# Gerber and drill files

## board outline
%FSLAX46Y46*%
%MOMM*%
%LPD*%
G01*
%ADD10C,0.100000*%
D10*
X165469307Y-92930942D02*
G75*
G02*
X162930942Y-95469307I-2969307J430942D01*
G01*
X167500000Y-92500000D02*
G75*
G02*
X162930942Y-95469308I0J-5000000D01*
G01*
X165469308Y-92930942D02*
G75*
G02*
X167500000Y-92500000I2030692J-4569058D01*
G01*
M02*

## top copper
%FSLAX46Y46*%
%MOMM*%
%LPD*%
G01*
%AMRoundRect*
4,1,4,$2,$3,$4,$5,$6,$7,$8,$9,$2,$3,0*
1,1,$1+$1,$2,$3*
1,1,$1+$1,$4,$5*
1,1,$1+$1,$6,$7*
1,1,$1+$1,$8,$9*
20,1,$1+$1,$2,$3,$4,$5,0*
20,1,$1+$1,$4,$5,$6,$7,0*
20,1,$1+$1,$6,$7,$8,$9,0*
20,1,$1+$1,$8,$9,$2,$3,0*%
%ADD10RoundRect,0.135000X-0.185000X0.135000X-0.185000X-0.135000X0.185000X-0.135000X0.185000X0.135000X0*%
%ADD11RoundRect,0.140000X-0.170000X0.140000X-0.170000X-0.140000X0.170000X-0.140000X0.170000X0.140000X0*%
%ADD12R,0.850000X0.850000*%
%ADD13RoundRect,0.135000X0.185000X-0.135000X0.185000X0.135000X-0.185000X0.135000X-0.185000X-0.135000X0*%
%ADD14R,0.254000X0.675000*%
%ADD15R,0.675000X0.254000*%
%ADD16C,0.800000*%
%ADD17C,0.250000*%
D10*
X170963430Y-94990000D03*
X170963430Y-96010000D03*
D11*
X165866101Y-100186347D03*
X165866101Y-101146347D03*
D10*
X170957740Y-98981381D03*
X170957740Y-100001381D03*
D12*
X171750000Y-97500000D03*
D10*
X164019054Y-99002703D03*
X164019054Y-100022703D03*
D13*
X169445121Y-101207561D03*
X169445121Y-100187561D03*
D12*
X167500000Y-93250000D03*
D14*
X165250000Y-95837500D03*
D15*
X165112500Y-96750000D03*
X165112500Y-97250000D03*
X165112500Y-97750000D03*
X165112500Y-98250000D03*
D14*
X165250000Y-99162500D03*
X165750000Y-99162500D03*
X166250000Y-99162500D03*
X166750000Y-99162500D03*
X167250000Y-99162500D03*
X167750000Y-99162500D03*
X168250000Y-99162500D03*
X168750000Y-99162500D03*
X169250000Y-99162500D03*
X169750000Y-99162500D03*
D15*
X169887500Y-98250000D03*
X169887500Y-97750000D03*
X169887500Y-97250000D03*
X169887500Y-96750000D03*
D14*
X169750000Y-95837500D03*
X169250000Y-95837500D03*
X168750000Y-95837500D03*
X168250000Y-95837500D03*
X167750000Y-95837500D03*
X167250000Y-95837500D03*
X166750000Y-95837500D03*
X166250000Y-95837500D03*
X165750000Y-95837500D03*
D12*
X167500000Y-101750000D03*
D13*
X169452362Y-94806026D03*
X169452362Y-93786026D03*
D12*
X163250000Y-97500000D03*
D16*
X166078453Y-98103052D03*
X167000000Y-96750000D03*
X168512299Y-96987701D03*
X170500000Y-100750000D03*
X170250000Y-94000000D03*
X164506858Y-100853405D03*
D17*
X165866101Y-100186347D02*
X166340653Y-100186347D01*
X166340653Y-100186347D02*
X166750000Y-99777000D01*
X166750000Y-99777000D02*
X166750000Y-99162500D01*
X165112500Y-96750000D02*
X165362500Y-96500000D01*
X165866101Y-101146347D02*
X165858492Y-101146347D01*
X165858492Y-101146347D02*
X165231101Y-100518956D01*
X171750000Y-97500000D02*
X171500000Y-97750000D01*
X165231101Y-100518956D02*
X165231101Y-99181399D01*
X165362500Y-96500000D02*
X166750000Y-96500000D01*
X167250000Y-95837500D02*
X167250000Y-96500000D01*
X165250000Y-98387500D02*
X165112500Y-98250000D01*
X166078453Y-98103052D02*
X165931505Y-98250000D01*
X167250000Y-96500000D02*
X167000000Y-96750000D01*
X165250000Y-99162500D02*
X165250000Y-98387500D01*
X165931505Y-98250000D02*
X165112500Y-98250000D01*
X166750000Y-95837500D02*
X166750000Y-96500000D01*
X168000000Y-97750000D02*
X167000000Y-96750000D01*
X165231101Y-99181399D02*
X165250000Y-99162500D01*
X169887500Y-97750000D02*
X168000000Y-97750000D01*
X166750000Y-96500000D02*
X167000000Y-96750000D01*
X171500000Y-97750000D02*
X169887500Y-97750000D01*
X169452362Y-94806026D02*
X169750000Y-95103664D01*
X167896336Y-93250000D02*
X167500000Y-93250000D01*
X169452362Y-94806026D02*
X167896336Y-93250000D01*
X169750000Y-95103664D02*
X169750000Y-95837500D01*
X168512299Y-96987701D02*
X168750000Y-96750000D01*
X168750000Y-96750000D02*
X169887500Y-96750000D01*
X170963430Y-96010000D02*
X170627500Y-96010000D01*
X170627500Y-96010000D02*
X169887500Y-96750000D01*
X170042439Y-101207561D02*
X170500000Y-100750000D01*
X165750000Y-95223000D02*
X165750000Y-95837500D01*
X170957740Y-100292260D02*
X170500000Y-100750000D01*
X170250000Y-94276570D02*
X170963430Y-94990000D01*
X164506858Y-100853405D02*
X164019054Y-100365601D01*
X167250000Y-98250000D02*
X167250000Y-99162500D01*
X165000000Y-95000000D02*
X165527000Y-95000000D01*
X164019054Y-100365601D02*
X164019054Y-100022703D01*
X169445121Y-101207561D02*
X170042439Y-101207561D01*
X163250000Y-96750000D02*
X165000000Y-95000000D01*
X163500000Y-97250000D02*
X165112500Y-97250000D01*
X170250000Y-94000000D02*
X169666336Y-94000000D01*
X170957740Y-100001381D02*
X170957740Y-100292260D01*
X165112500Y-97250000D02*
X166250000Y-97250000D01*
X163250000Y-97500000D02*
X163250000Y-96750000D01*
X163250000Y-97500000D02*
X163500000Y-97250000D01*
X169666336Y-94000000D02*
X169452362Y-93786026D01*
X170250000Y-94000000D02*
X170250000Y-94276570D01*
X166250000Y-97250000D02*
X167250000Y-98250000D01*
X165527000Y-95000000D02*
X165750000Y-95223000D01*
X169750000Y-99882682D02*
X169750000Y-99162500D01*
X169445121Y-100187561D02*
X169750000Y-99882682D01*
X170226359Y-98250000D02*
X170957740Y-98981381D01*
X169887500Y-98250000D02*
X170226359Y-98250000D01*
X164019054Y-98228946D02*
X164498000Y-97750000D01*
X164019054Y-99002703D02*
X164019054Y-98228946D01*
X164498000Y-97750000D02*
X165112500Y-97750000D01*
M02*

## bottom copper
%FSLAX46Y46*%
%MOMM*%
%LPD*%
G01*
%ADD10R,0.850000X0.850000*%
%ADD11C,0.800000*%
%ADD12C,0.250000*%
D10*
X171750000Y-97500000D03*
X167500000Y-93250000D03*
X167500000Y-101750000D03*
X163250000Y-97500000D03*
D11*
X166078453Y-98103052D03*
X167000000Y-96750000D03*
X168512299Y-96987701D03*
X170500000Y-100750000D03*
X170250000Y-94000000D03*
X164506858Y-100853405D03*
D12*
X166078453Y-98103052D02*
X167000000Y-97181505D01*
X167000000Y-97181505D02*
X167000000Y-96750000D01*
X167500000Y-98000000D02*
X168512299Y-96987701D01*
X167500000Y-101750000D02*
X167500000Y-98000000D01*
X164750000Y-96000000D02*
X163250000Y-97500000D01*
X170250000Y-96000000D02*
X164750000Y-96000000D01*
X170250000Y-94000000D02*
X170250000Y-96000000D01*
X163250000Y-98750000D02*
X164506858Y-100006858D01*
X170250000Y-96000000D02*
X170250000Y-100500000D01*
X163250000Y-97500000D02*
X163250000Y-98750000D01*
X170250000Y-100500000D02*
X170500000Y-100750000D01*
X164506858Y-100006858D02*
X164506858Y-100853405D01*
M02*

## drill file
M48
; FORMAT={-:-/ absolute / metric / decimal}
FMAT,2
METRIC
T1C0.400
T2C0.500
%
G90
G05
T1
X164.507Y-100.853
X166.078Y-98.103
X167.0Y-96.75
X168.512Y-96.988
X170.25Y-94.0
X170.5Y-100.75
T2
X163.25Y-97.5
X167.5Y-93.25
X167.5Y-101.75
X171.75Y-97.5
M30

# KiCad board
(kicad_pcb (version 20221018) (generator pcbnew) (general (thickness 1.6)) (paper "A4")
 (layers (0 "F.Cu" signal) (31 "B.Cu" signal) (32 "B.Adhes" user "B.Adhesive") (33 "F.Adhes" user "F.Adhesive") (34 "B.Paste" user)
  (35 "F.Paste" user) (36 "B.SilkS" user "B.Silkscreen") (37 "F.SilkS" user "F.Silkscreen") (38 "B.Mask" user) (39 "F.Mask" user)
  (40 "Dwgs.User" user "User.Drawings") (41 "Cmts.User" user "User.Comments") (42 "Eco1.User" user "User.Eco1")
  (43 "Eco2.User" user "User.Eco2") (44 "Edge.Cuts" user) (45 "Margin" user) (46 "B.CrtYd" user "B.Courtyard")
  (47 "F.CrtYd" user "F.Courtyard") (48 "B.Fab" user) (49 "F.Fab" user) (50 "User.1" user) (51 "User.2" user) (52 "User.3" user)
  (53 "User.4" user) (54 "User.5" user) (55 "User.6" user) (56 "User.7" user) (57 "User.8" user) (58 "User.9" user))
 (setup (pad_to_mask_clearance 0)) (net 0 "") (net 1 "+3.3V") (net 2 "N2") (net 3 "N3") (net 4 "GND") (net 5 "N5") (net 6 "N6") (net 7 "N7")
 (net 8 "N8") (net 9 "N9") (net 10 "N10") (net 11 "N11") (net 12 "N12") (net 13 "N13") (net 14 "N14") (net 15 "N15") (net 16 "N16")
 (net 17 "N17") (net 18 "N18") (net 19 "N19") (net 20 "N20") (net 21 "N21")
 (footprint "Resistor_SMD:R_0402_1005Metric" (layer "F.Cu") (at 170.96343 95.5 -90)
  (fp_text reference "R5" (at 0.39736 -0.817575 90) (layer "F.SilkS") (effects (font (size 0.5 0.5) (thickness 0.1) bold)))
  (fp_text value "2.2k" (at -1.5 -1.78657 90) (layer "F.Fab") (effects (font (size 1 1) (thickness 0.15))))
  (pad "1" smd roundrect (at -0.51 0 270) (size 0.54 0.64) (layers "F.Cu" "F.Paste" "F.Mask") (roundrect_rratio 0.25) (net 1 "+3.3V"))
  (pad "2" smd roundrect (at 0.51 0 270) (size 0.54 0.64) (layers "F.Cu" "F.Paste" "F.Mask") (roundrect_rratio 0.25) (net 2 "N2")))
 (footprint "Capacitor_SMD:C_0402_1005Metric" (layer "F.Cu") (at 165.866101 100.666347 -90)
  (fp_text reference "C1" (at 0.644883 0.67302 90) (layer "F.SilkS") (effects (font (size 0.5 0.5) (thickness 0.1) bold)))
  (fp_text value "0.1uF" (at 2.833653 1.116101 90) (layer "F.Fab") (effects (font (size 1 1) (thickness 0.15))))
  (pad "1" smd roundrect (at -0.48 0 270) (size 0.56 0.62) (layers "F.Cu" "F.Paste" "F.Mask") (roundrect_rratio 0.25) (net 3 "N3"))
  (pad "2" smd roundrect (at 0.48 0 270) (size 0.56 0.62) (layers "F.Cu" "F.Paste" "F.Mask") (roundrect_rratio 0.25) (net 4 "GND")))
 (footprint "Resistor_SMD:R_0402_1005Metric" (layer "F.Cu") (at 170.95774 99.491381 -90)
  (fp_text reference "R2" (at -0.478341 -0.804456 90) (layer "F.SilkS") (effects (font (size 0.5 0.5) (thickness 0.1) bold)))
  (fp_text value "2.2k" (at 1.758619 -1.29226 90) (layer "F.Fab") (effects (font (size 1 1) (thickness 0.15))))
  (pad "1" smd roundrect (at -0.51 0 270) (size 0.54 0.64) (layers "F.Cu" "F.Paste" "F.Mask") (roundrect_rratio 0.25) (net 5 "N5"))
  (pad "2" smd roundrect (at 0.51 0 270) (size 0.54 0.64) (layers "F.Cu" "F.Paste" "F.Mask") (roundrect_rratio 0.25) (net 1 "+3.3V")))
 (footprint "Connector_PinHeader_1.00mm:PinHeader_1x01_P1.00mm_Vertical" (layer "F.Cu") (at 171.75 97.5)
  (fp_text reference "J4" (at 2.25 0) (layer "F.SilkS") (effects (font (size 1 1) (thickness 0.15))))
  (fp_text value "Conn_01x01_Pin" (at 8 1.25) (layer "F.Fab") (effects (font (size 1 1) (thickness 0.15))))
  (pad "1" thru_hole rect (at 0 0) (size 0.85 0.85) (drill 0.5) (layers "*.Cu" "*.Mask") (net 4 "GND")))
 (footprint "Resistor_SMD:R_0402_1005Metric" (layer "F.Cu") (at 164.019054 99.512703 -90)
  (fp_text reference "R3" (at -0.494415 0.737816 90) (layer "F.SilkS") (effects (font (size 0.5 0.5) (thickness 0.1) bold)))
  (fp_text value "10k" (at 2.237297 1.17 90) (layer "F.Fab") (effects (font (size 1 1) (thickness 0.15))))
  (pad "1" smd roundrect (at -0.51 0 270) (size 0.54 0.64) (layers "F.Cu" "F.Paste" "F.Mask") (roundrect_rratio 0.25) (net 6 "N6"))
  (pad "2" smd roundrect (at 0.51 0 270) (size 0.54 0.64) (layers "F.Cu" "F.Paste" "F.Mask") (roundrect_rratio 0.25) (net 1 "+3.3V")))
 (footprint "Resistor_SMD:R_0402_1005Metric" (layer "F.Cu") (at 169.445121 100.697561 90)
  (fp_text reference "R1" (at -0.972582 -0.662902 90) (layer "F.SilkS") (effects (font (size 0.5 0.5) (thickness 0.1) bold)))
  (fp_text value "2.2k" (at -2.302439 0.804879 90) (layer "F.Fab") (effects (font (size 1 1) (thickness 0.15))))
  (pad "1" smd roundrect (at -0.51 0 90) (size 0.54 0.64) (layers "F.Cu" "F.Paste" "F.Mask") (roundrect_rratio 0.25) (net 1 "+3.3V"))
  (pad "2" smd roundrect (at 0.51 0 90) (size 0.54 0.64) (layers "F.Cu" "F.Paste" "F.Mask") (roundrect_rratio 0.25) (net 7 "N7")))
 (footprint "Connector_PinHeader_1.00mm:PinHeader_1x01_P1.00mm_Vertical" (layer "F.Cu") (at 167.5 93.25)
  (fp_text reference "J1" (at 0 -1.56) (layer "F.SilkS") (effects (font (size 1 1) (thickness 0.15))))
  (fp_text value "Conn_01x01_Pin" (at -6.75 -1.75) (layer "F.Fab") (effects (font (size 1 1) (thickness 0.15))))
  (pad "1" thru_hole rect (at 0 0) (size 0.85 0.85) (drill 0.5) (layers "*.Cu" "*.Mask") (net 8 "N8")))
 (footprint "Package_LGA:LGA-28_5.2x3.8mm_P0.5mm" (layer "F.Cu") (at 167.5 97.5)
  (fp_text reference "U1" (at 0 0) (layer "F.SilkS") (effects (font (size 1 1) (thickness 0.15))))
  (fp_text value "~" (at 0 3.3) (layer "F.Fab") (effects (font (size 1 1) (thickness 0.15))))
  (pad "1" smd rect (at -2.25 -1.6625) (size 0.254 0.675) (layers "F.Cu" "F.Paste" "F.Mask") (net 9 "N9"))
  (pad "2" smd rect (at -2.3875 -0.75 90) (size 0.254 0.675) (layers "F.Cu" "F.Paste" "F.Mask") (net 4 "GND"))
  (pad "3" smd rect (at -2.3875 -0.25 90) (size 0.254 0.675) (layers "F.Cu" "F.Paste" "F.Mask") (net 1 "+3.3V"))
  (pad "4" smd rect (at -2.3875 0.25 90) (size 0.254 0.675) (layers "F.Cu" "F.Paste" "F.Mask") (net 6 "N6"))
  (pad "5" smd rect (at -2.3875 0.75 90) (size 0.254 0.675) (layers "F.Cu" "F.Paste" "F.Mask") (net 4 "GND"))
  (pad "6" smd rect (at -2.25 1.6625) (size 0.254 0.675) (layers "F.Cu" "F.Paste" "F.Mask") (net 4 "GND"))
  (pad "7" smd rect (at -1.75 1.6625) (size 0.254 0.675) (layers "F.Cu" "F.Paste" "F.Mask") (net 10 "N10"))
  (pad "8" smd rect (at -1.25 1.6625) (size 0.254 0.675) (layers "F.Cu" "F.Paste" "F.Mask") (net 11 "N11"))
  (pad "9" smd rect (at -0.75 1.6625) (size 0.254 0.675) (layers "F.Cu" "F.Paste" "F.Mask") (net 3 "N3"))
  (pad "10" smd rect (at -0.25 1.6625) (size 0.254 0.675) (layers "F.Cu" "F.Paste" "F.Mask") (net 1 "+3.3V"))
  (pad "11" smd rect (at 0.25 1.6625) (size 0.254 0.675) (layers "F.Cu" "F.Paste" "F.Mask") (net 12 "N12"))
  (pad "12" smd rect (at 0.75 1.6625) (size 0.254 0.675) (layers "F.Cu" "F.Paste" "F.Mask") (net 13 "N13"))
  (pad "13" smd rect (at 1.25 1.6625) (size 0.254 0.675) (layers "F.Cu" "F.Paste" "F.Mask") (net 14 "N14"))
  (pad "14" smd rect (at 1.75 1.6625) (size 0.254 0.675) (layers "F.Cu" "F.Paste" "F.Mask") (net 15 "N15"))
  (pad "15" smd rect (at 2.25 1.6625) (size 0.254 0.675) (layers "F.Cu" "F.Paste" "F.Mask") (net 7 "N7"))
  (pad "16" smd rect (at 2.3875 0.75 90) (size 0.254 0.675) (layers "F.Cu" "F.Paste" "F.Mask") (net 5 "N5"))
  (pad "17" smd rect (at 2.3875 0.25 90) (size 0.254 0.675) (layers "F.Cu" "F.Paste" "F.Mask") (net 4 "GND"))
  (pad "18" smd rect (at 2.3875 -0.25 90) (size 0.254 0.675) (layers "F.Cu" "F.Paste" "F.Mask") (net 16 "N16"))
  (pad "19" smd rect (at 2.3875 -0.75 90) (size 0.254 0.675) (layers "F.Cu" "F.Paste" "F.Mask") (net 2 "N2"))
  (pad "20" smd rect (at 2.25 -1.6625) (size 0.254 0.675) (layers "F.Cu" "F.Paste" "F.Mask") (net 8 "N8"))
  (pad "21" smd rect (at 1.75 -1.6625) (size 0.254 0.675) (layers "F.Cu" "F.Paste" "F.Mask") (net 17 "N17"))
  (pad "22" smd rect (at 1.25 -1.6625) (size 0.254 0.675) (layers "F.Cu" "F.Paste" "F.Mask") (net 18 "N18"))
  (pad "23" smd rect (at 0.75 -1.6625) (size 0.254 0.675) (layers "F.Cu" "F.Paste" "F.Mask") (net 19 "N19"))
  (pad "24" smd rect (at 0.25 -1.6625) (size 0.254 0.675) (layers "F.Cu" "F.Paste" "F.Mask") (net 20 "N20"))
  (pad "25" smd rect (at -0.25 -1.6625) (size 0.254 0.675) (layers "F.Cu" "F.Paste" "F.Mask") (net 4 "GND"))
  (pad "26" smd rect (at -0.75 -1.6625) (size 0.254 0.675) (layers "F.Cu" "F.Paste" "F.Mask") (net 4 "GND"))
  (pad "27" smd rect (at -1.25 -1.6625) (size 0.254 0.675) (layers "F.Cu" "F.Paste" "F.Mask") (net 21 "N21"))
  (pad "28" smd rect (at -1.75 -1.6625) (size 0.254 0.675) (layers "F.Cu" "F.Paste" "F.Mask") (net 1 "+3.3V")))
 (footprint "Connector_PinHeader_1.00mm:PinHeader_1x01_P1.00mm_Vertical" (layer "F.Cu") (at 167.5 101.75)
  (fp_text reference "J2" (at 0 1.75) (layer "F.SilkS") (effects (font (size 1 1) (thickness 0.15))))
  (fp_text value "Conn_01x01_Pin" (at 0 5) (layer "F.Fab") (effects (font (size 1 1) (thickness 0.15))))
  (pad "1" thru_hole rect (at 0 0) (size 0.85 0.85) (drill 0.5) (layers "*.Cu" "*.Mask") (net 2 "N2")))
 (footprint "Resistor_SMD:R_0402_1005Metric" (layer "F.Cu") (at 169.452362 94.296026 90)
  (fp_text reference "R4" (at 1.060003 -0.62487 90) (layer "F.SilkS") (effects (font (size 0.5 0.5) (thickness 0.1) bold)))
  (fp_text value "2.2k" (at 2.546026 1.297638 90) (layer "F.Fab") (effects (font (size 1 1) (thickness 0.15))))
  (pad "1" smd roundrect (at -0.51 0 90) (size 0.54 0.64) (layers "F.Cu" "F.Paste" "F.Mask") (roundrect_rratio 0.25) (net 8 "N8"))
  (pad "2" smd roundrect (at 0.51 0 90) (size 0.54 0.64) (layers "F.Cu" "F.Paste" "F.Mask") (roundrect_rratio 0.25) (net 1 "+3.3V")))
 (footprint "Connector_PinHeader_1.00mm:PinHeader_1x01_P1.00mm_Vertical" (layer "F.Cu") (at 163.25 97.5)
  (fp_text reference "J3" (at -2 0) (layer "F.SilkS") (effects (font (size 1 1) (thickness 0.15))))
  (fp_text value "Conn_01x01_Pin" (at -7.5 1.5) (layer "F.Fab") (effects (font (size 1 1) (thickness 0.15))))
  (pad "1" thru_hole rect (at 0 0) (size 0.85 0.85) (drill 0.5) (layers "*.Cu" "*.Mask") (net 1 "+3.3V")))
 (gr_arc (start 165.469307 92.930942) (mid 164.621614 94.621614) (end 162.930942 95.469307) (stroke (width 0.1) (type default))
  (layer "Edge.Cuts"))
 (gr_arc (start 167.5 92.5) (mid 170.224568 101.692461) (end 162.930942 95.469308) (stroke (width 0.1) (type default)) (layer "Edge.Cuts"))
 (gr_arc (start 165.469308 92.930942) (mid 166.462043 92.608922) (end 167.5 92.5) (stroke (width 0.1) (type default)) (layer "Edge.Cuts"))
 (segment (start 165.866101 100.186347) (end 166.340653 100.186347) (width 0.25) (layer "F.Cu") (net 3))
 (segment (start 166.340653 100.186347) (end 166.75 99.777) (width 0.25) (layer "F.Cu") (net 3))
 (segment (start 166.75 99.777) (end 166.75 99.1625) (width 0.25) (layer "F.Cu") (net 3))
 (segment (start 165.1125 96.75) (end 165.3625 96.5) (width 0.25) (layer "F.Cu") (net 4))
 (segment (start 165.866101 101.146347) (end 165.858492 101.146347) (width 0.25) (layer "F.Cu") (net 4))
 (segment (start 165.858492 101.146347) (end 165.231101 100.518956) (width 0.25) (layer "F.Cu") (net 4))
 (segment (start 171.75 97.5) (end 171.5 97.75) (width 0.25) (layer "F.Cu") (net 4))
 (segment (start 165.231101 100.518956) (end 165.231101 99.181399) (width 0.25) (layer "F.Cu") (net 4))
 (segment (start 165.3625 96.5) (end 166.75 96.5) (width 0.25) (layer "F.Cu") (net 4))
 (segment (start 167.25 95.8375) (end 167.25 96.5) (width 0.25) (layer "F.Cu") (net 4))
 (segment (start 165.25 98.3875) (end 165.1125 98.25) (width 0.25) (layer "F.Cu") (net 4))
 (segment (start 166.078453 98.103052) (end 165.931505 98.25) (width 0.25) (layer "F.Cu") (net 4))
 (segment (start 167.25 96.5) (end 167 96.75) (width 0.25) (layer "F.Cu") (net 4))
 (segment (start 165.25 99.1625) (end 165.25 98.3875) (width 0.25) (layer "F.Cu") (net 4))
 (segment (start 165.931505 98.25) (end 165.1125 98.25) (width 0.25) (layer "F.Cu") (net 4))
 (segment (start 166.75 95.8375) (end 166.75 96.5) (width 0.25) (layer "F.Cu") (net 4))
 (segment (start 168 97.75) (end 167 96.75) (width 0.25) (layer "F.Cu") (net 4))
 (segment (start 165.231101 99.181399) (end 165.25 99.1625) (width 0.25) (layer "F.Cu") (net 4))
 (segment (start 169.8875 97.75) (end 168 97.75) (width 0.25) (layer "F.Cu") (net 4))
 (segment (start 166.75 96.5) (end 167 96.75) (width 0.25) (layer "F.Cu") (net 4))
 (segment (start 171.5 97.75) (end 169.8875 97.75) (width 0.25) (layer "F.Cu") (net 4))
 (via (at 166.078453 98.103052) (size 0.8) (drill 0.4) (layers "F.Cu" "B.Cu") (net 4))
 (via (at 167 96.75) (size 0.8) (drill 0.4) (layers "F.Cu" "B.Cu") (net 4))
 (segment (start 166.078453 98.103052) (end 167 97.181505) (width 0.25) (layer "B.Cu") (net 4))
 (segment (start 167 97.181505) (end 167 96.75) (width 0.25) (layer "B.Cu") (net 4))
 (segment (start 169.452362 94.806026) (end 169.75 95.103664) (width 0.25) (layer "F.Cu") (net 8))
 (segment (start 167.896336 93.25) (end 167.5 93.25) (width 0.25) (layer "F.Cu") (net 8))
 (segment (start 169.452362 94.806026) (end 167.896336 93.25) (width 0.25) (layer "F.Cu") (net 8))
 (segment (start 169.75 95.103664) (end 169.75 95.8375) (width 0.25) (layer "F.Cu") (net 8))
 (segment (start 168.512299 96.987701) (end 168.75 96.75) (width 0.25) (layer "F.Cu") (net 2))
 (segment (start 168.75 96.75) (end 169.8875 96.75) (width 0.25) (layer "F.Cu") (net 2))
 (segment (start 170.96343 96.01) (end 170.6275 96.01) (width 0.25) (layer "F.Cu") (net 2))
 (segment (start 170.6275 96.01) (end 169.8875 96.75) (width 0.25) (layer "F.Cu") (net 2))
 (via (at 168.512299 96.987701) (size 0.8) (drill 0.4) (layers "F.Cu" "B.Cu") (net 2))
 (segment (start 167.5 98) (end 168.512299 96.987701) (width 0.25) (layer "B.Cu") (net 2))
 (segment (start 167.5 101.75) (end 167.5 98) (width 0.25) (layer "B.Cu") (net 2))
 (segment (start 170.042439 101.207561) (end 170.5 100.75) (width 0.25) (layer "F.Cu") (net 1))
 (segment (start 165.75 95.223) (end 165.75 95.8375) (width 0.25) (layer "F.Cu") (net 1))
 (segment (start 170.95774 100.29226) (end 170.5 100.75) (width 0.25) (layer "F.Cu") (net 1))
 (segment (start 170.25 94.27657) (end 170.96343 94.99) (width 0.25) (layer "F.Cu") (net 1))
 (segment (start 164.506858 100.853405) (end 164.019054 100.365601) (width 0.25) (layer "F.Cu") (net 1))
 (segment (start 167.25 98.25) (end 167.25 99.1625) (width 0.25) (layer "F.Cu") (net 1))
 (segment (start 165 95) (end 165.527 95) (width 0.25) (layer "F.Cu") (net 1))
 (segment (start 164.019054 100.365601) (end 164.019054 100.022703) (width 0.25) (layer "F.Cu") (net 1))
 (segment (start 169.445121 101.207561) (end 170.042439 101.207561) (width 0.25) (layer "F.Cu") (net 1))
 (segment (start 163.25 96.75) (end 165 95) (width 0.25) (layer "F.Cu") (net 1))
 (segment (start 163.5 97.25) (end 165.1125 97.25) (width 0.25) (layer "F.Cu") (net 1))
 (segment (start 170.25 94) (end 169.666336 94) (width 0.25) (layer "F.Cu") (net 1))
 (segment (start 170.95774 100.001381) (end 170.95774 100.29226) (width 0.25) (layer "F.Cu") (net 1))
 (segment (start 165.1125 97.25) (end 166.25 97.25) (width 0.25) (layer "F.Cu") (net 1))
 (segment (start 163.25 97.5) (end 163.25 96.75) (width 0.25) (layer "F.Cu") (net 1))
 (segment (start 163.25 97.5) (end 163.5 97.25) (width 0.25) (layer "F.Cu") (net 1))
 (segment (start 169.666336 94) (end 169.452362 93.786026) (width 0.25) (layer "F.Cu") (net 1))
 (segment (start 170.25 94) (end 170.25 94.27657) (width 0.25) (layer "F.Cu") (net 1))
 (segment (start 166.25 97.25) (end 167.25 98.25) (width 0.25) (layer "F.Cu") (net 1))
 (segment (start 165.527 95) (end 165.75 95.223) (width 0.25) (layer "F.Cu") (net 1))
 (via (at 170.5 100.75) (size 0.8) (drill 0.4) (layers "F.Cu" "B.Cu") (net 1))
 (via (at 170.25 94) (size 0.8) (drill 0.4) (layers "F.Cu" "B.Cu") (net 1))
 (via (at 164.506858 100.853405) (size 0.8) (drill 0.4) (layers "F.Cu" "B.Cu") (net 1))
 (segment (start 164.75 96) (end 163.25 97.5) (width 0.25) (layer "B.Cu") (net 1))
 (segment (start 170.25 96) (end 164.75 96) (width 0.25) (layer "B.Cu") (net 1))
 (segment (start 170.25 94) (end 170.25 96) (width 0.25) (layer "B.Cu") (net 1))
 (segment (start 163.25 98.75) (end 164.506858 100.006858) (width 0.25) (layer "B.Cu") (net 1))
 (segment (start 170.25 96) (end 170.25 100.5) (width 0.25) (layer "B.Cu") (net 1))
 (segment (start 163.25 97.5) (end 163.25 98.75) (width 0.25) (layer "B.Cu") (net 1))
 (segment (start 170.25 100.5) (end 170.5 100.75) (width 0.25) (layer "B.Cu") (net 1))
 (segment (start 164.506858 100.006858) (end 164.506858 100.853405) (width 0.25) (layer "B.Cu") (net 1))
 (segment (start 169.75 99.882682) (end 169.75 99.1625) (width 0.25) (layer "F.Cu") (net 7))
 (segment (start 169.445121 100.187561) (end 169.75 99.882682) (width 0.25) (layer "F.Cu") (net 7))
 (segment (start 170.226359 98.25) (end 170.95774 98.981381) (width 0.25) (layer "F.Cu") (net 5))
 (segment (start 169.8875 98.25) (end 170.226359 98.25) (width 0.25) (layer "F.Cu") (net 5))
 (segment (start 164.019054 98.228946) (end 164.498 97.75) (width 0.25) (layer "F.Cu") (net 6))
 (segment (start 164.019054 99.002703) (end 164.019054 98.228946) (width 0.25) (layer "F.Cu") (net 6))
 (segment (start 164.498 97.75) (end 165.1125 97.75) (width 0.25) (layer "F.Cu") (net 6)))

